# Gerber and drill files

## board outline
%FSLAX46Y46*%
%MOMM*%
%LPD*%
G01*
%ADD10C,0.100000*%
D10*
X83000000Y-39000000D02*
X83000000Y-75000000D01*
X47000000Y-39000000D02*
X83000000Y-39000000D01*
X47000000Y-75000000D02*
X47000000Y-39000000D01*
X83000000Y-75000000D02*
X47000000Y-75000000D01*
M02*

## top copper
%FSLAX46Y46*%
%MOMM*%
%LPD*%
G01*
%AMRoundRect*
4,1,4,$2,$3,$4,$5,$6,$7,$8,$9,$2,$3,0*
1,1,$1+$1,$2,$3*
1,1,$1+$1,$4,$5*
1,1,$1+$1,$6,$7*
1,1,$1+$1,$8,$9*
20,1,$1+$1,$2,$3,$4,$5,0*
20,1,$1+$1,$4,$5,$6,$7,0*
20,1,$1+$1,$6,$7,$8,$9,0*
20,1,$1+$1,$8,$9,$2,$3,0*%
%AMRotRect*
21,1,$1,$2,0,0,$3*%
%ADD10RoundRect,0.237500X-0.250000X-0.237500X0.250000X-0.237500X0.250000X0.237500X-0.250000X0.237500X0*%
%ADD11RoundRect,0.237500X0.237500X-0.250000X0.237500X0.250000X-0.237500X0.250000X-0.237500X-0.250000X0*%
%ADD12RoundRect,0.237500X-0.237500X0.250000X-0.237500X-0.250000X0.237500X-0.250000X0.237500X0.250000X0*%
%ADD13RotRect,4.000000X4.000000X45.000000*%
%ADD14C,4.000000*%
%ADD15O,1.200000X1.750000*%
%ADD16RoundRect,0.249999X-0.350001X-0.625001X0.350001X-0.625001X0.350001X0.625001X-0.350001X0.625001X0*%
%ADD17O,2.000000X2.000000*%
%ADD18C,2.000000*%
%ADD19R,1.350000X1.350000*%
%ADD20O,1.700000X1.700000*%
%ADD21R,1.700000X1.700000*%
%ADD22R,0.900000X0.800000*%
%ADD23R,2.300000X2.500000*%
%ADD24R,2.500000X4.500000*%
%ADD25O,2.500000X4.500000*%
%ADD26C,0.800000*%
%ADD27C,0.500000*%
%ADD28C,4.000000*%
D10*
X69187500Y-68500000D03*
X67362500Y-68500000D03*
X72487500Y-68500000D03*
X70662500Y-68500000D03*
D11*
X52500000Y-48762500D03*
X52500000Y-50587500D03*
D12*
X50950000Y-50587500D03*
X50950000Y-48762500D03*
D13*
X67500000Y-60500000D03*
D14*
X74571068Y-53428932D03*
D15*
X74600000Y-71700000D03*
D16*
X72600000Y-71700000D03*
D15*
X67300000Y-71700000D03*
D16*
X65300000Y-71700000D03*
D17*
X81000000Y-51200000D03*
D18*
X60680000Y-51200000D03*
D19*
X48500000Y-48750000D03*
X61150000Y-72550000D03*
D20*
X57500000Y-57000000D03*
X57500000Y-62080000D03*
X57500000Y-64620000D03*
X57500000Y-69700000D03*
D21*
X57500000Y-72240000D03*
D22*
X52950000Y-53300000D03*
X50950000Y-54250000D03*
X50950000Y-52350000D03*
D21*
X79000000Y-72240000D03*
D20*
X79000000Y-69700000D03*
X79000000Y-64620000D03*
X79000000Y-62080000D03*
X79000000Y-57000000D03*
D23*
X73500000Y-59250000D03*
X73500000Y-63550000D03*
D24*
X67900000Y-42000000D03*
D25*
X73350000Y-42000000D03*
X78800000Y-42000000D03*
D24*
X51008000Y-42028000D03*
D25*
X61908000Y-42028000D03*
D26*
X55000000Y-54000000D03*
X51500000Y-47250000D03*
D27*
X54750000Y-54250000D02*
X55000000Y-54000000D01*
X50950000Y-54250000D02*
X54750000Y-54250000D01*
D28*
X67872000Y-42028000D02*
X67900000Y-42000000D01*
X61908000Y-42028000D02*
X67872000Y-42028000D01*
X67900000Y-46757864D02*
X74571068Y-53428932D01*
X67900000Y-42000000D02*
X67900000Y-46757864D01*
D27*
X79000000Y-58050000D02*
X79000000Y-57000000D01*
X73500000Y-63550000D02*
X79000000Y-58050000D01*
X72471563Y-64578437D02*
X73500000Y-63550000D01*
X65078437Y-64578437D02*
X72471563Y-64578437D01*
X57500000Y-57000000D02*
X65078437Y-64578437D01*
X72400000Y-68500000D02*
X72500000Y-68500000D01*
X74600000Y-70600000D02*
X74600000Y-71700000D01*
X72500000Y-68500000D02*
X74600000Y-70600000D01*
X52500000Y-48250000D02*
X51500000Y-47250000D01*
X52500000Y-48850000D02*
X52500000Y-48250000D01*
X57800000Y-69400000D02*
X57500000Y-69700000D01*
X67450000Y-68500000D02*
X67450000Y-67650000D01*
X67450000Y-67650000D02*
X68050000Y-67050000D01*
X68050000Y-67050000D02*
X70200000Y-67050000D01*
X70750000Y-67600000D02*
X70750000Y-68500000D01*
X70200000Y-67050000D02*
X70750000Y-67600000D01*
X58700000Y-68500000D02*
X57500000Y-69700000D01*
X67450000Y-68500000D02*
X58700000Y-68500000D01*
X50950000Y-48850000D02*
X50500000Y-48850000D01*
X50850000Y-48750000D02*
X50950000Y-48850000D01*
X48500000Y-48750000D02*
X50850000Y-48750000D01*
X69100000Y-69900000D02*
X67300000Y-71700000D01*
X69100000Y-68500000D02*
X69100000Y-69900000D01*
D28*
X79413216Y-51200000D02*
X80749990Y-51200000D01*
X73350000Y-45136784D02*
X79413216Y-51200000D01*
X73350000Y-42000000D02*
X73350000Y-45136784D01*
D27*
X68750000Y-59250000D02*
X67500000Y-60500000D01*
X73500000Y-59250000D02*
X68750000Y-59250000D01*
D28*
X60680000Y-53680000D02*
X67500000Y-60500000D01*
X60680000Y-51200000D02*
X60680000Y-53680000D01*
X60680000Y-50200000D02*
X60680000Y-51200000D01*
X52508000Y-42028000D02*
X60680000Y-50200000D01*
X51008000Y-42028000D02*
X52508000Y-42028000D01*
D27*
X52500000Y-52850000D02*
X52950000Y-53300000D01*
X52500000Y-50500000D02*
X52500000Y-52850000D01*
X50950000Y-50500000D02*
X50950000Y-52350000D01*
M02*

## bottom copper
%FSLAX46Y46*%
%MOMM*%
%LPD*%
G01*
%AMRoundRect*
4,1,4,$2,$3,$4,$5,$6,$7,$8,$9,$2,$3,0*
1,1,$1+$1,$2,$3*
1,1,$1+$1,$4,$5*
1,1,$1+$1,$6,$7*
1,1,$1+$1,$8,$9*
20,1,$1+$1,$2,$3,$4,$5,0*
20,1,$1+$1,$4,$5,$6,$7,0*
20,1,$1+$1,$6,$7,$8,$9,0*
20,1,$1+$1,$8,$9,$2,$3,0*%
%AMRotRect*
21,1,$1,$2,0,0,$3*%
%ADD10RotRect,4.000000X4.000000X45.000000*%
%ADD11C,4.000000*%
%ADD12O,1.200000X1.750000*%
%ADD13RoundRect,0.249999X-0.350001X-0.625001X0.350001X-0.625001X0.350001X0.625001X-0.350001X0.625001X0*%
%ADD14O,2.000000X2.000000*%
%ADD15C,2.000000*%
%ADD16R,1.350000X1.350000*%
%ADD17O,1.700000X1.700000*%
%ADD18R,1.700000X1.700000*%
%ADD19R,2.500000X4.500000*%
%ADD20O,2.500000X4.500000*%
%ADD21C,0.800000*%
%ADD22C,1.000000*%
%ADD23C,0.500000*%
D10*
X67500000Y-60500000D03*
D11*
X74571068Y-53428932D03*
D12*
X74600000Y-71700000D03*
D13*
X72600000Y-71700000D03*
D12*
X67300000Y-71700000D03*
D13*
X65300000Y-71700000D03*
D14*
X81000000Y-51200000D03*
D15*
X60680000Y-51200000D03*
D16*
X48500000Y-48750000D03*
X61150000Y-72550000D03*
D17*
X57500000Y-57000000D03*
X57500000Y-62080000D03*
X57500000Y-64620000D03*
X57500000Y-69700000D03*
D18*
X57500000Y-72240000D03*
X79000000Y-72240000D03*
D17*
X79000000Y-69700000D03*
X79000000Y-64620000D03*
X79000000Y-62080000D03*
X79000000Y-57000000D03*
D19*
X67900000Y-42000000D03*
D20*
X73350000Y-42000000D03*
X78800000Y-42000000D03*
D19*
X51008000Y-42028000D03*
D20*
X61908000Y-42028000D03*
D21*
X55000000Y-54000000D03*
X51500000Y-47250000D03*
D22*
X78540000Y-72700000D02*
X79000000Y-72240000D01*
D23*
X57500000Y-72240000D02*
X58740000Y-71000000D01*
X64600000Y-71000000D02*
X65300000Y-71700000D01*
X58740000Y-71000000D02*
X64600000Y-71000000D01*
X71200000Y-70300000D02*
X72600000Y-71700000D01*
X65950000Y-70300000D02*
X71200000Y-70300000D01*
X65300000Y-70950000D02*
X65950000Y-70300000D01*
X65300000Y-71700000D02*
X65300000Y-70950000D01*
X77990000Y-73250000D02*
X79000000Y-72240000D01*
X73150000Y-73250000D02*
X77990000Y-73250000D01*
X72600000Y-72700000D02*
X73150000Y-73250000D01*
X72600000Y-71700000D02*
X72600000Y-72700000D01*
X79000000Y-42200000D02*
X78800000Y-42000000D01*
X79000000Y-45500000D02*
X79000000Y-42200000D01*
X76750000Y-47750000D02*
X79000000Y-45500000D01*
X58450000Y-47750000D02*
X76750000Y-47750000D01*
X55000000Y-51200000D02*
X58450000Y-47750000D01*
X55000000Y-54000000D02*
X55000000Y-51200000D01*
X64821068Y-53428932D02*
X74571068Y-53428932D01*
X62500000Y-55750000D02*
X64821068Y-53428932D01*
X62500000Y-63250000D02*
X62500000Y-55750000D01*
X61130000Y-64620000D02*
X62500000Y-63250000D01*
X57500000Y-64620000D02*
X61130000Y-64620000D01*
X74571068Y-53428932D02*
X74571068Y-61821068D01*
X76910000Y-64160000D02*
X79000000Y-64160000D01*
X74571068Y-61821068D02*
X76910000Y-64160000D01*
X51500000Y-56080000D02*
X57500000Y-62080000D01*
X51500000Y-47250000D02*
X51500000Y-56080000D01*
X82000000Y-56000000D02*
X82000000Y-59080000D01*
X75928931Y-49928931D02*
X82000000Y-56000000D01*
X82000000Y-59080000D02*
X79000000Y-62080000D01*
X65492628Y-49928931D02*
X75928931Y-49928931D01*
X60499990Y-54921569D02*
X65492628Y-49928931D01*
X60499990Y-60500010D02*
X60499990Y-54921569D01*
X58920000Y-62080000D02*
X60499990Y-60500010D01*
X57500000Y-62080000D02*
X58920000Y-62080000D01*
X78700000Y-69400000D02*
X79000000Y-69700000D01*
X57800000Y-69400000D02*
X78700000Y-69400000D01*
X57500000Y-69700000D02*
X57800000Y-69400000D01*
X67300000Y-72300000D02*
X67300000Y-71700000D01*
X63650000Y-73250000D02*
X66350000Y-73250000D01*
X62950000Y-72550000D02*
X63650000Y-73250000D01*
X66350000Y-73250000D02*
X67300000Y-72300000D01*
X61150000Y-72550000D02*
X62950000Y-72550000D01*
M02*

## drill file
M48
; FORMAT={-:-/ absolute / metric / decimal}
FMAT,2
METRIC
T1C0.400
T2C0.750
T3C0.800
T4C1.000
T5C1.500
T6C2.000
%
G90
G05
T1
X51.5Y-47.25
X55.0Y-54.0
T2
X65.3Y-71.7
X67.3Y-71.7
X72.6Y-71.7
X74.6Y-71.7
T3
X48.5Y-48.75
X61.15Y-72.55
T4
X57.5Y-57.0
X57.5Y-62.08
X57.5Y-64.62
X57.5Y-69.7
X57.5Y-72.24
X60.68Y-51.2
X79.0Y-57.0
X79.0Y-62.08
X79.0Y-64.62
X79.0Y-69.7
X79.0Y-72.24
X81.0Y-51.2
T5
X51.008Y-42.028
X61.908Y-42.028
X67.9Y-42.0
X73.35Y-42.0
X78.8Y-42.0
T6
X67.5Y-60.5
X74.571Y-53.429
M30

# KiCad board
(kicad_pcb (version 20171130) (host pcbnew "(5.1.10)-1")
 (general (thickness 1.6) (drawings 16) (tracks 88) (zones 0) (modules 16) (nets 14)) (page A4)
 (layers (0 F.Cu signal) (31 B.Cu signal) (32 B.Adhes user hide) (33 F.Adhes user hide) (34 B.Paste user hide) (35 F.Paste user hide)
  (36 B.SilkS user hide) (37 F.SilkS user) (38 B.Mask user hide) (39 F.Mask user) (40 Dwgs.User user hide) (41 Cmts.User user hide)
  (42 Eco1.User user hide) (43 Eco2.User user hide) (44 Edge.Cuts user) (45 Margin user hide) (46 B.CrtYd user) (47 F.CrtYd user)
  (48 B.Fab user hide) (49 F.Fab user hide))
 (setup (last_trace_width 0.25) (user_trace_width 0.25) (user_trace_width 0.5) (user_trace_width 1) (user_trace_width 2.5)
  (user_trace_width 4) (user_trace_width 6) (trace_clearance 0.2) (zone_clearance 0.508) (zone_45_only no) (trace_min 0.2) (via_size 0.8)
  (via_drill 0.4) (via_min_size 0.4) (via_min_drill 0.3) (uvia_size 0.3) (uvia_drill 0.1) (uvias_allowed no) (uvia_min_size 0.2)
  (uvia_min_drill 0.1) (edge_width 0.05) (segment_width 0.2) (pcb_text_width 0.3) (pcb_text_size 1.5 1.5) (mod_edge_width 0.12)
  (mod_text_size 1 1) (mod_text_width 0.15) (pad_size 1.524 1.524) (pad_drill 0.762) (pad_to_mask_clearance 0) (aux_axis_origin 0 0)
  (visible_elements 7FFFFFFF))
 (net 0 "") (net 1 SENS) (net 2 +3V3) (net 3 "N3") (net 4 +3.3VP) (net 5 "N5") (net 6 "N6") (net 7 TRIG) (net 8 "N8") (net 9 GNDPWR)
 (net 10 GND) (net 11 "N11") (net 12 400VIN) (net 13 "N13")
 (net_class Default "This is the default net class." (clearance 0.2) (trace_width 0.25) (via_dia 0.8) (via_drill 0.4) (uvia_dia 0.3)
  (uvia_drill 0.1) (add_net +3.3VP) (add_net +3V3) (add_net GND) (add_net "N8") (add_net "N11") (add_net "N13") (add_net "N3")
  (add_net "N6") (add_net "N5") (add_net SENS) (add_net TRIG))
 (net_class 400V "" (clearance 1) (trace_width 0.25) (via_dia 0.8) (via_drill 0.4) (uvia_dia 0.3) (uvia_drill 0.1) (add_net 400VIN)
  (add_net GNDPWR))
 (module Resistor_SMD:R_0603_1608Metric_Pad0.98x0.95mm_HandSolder (layer F.Cu) (at 68.275 68.5)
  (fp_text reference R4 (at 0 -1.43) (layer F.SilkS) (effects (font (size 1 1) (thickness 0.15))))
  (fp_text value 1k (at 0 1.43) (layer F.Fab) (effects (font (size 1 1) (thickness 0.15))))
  (pad 2 smd roundrect (at 0.9125 0) (size 0.975 0.95) (layers F.Cu F.Paste F.Mask) (roundrect_rratio 0.25) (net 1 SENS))
  (pad 1 smd roundrect (at -0.9125 0) (size 0.975 0.95) (layers F.Cu F.Paste F.Mask) (roundrect_rratio 0.25) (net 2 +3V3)))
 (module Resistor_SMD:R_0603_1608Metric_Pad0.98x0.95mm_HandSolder (layer F.Cu) (at 71.575 68.5)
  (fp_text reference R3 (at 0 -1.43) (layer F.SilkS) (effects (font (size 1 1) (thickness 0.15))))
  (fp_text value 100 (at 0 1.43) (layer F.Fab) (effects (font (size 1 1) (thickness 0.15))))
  (pad 2 smd roundrect (at 0.9125 0) (size 0.975 0.95) (layers F.Cu F.Paste F.Mask) (roundrect_rratio 0.25) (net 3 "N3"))
  (pad 1 smd roundrect (at -0.9125 0) (size 0.975 0.95) (layers F.Cu F.Paste F.Mask) (roundrect_rratio 0.25) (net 2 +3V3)))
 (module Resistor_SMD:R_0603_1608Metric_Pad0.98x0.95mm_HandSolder (layer F.Cu) (at 52.5 49.675 90)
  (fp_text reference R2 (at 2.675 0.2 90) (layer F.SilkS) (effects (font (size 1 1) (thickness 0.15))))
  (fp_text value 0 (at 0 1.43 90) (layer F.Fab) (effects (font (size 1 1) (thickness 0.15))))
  (pad 2 smd roundrect (at 0.9125 0 90) (size 0.975 0.95) (layers F.Cu F.Paste F.Mask) (roundrect_rratio 0.25) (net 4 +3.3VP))
  (pad 1 smd roundrect (at -0.9125 0 90) (size 0.975 0.95) (layers F.Cu F.Paste F.Mask) (roundrect_rratio 0.25) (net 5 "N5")))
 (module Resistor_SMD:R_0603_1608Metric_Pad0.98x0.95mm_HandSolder (layer F.Cu) (at 50.95 49.675 270)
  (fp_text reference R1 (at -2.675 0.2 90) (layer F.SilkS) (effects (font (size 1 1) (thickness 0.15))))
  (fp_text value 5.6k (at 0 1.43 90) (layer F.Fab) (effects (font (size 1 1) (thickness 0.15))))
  (pad 2 smd roundrect (at 0.9125 0 270) (size 0.975 0.95) (layers F.Cu F.Paste F.Mask) (roundrect_rratio 0.25) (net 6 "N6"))
  (pad 1 smd roundrect (at -0.9125 0 270) (size 0.975 0.95) (layers F.Cu F.Paste F.Mask) (roundrect_rratio 0.25) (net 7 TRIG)))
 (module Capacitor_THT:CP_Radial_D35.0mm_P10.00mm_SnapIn (layer B.Cu) (at 67.5 60.5 45)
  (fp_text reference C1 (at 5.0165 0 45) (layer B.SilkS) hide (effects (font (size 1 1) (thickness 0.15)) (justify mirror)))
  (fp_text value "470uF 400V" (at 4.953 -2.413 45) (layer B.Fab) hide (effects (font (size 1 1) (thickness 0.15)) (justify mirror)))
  (pad 1 thru_hole rect (at 0 0 45) (size 4 4) (drill 2) (layers *.Cu *.Mask) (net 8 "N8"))
  (pad 2 thru_hole circle (at 10 0 45) (size 4 4) (drill 2) (layers *.Cu *.Mask) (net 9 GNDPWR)))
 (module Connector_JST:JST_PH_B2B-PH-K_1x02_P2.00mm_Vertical (layer F.Cu) (at 72.6 71.7)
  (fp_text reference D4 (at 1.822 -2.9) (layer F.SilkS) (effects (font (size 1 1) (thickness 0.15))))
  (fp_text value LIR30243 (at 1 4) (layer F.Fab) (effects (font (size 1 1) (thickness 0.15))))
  (pad 2 thru_hole oval (at 2 0) (size 1.2 1.75) (drill 0.75) (layers *.Cu *.Mask) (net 3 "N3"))
  (pad 1 thru_hole roundrect (at 0 0) (size 1.2 1.75) (drill 0.75) (layers *.Cu *.Mask) (roundrect_rratio 0.2083325) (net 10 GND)))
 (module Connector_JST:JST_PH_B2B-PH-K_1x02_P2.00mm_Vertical (layer F.Cu) (at 65.3 71.7)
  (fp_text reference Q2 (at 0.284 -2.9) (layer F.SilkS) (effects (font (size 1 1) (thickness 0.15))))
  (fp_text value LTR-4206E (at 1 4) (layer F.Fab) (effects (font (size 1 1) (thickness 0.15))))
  (pad 2 thru_hole oval (at 2 0) (size 1.2 1.75) (drill 0.75) (layers *.Cu *.Mask) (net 1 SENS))
  (pad 1 thru_hole roundrect (at 0 0) (size 1.2 1.75) (drill 0.75) (layers *.Cu *.Mask) (roundrect_rratio 0.2083325) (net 10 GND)))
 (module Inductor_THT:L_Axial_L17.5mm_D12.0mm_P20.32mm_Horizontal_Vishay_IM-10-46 (layer F.Cu) (at 60.68 51.2)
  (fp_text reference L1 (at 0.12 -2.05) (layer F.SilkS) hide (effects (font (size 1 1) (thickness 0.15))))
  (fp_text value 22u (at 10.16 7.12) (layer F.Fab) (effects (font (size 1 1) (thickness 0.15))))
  (pad 2 thru_hole oval (at 20.32 0) (size 2 2) (drill 1) (layers *.Cu *.Mask) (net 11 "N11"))
  (pad 1 thru_hole circle (at 0 0) (size 2 2) (drill 1) (layers *.Cu *.Mask) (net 8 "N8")))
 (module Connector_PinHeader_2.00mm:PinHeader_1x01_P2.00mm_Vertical (layer F.Cu) (at 48.5 48.75 180)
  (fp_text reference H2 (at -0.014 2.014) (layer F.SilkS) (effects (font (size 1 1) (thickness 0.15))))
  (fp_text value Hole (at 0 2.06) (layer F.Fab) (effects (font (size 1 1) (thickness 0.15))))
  (pad 1 thru_hole rect (at 0 0 180) (size 1.35 1.35) (drill 0.8) (layers *.Cu *.Mask) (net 7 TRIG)))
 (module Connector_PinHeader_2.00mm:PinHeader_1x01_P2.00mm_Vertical (layer F.Cu) (at 61.15 72.55 180)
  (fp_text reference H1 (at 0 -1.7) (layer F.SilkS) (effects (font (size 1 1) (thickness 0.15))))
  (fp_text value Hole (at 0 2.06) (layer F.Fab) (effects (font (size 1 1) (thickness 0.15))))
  (pad 1 thru_hole rect (at 0 0 180) (size 1.35 1.35) (drill 0.8) (layers *.Cu *.Mask) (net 1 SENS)))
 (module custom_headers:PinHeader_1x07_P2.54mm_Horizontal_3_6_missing (layer F.Cu) (at 57.5 72.24 180)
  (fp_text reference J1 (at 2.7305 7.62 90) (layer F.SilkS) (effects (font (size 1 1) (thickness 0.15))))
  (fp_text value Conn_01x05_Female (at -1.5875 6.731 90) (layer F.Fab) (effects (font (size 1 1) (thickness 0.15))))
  (pad 5 thru_hole oval (at 0 15.24 180) (size 1.7 1.7) (drill 1) (layers *.Cu *.Mask) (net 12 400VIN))
  (pad 4 thru_hole oval (at 0 10.16 180) (size 1.7 1.7) (drill 1) (layers *.Cu *.Mask) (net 4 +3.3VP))
  (pad 3 thru_hole oval (at 0 7.62 180) (size 1.7 1.7) (drill 1) (layers *.Cu *.Mask) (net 9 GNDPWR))
  (pad 2 thru_hole oval (at 0 2.54 180) (size 1.7 1.7) (drill 1) (layers *.Cu *.Mask) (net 2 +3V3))
  (pad 1 thru_hole rect (at 0 0 180) (size 1.7 1.7) (drill 1) (layers *.Cu *.Mask) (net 10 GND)))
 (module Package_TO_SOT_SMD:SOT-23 (layer F.Cu) (at 51.95 53.3)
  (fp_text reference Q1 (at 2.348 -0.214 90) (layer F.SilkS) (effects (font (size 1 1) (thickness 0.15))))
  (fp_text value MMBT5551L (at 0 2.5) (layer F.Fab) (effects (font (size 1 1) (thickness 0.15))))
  (pad 3 smd rect (at 1 0) (size 0.9 0.8) (layers F.Cu F.Paste F.Mask) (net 5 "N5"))
  (pad 2 smd rect (at -1 0.95) (size 0.9 0.8) (layers F.Cu F.Paste F.Mask) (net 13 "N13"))
  (pad 1 smd rect (at -1 -0.95) (size 0.9 0.8) (layers F.Cu F.Paste F.Mask) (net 6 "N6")))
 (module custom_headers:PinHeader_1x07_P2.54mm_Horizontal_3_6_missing (layer B.Cu) (at 79 72.24)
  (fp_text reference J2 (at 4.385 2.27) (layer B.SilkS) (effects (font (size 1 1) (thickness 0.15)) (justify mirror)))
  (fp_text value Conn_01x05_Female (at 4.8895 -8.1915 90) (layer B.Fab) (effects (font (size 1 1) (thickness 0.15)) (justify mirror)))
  (pad 1 thru_hole rect (at 0 0) (size 1.7 1.7) (drill 1) (layers *.Cu *.Mask) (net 10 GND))
  (pad 2 thru_hole oval (at 0 -2.54) (size 1.7 1.7) (drill 1) (layers *.Cu *.Mask) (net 2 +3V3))
  (pad 3 thru_hole oval (at 0 -7.62) (size 1.7 1.7) (drill 1) (layers *.Cu *.Mask) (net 9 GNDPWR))
  (pad 4 thru_hole oval (at 0 -10.16) (size 1.7 1.7) (drill 1) (layers *.Cu *.Mask) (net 4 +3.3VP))
  (pad 5 thru_hole oval (at 0 -15.24) (size 1.7 1.7) (drill 1) (layers *.Cu *.Mask) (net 12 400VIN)))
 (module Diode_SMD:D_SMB (layer F.Cu) (at 73.5 61.4 270)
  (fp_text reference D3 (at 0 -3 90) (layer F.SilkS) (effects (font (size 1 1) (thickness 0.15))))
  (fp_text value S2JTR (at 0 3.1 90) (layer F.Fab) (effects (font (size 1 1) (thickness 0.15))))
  (pad 1 smd rect (at -2.15 0 270) (size 2.5 2.3) (layers F.Cu F.Paste F.Mask) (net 8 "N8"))
  (pad 2 smd rect (at 2.15 0 270) (size 2.5 2.3) (layers F.Cu F.Paste F.Mask) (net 12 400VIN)))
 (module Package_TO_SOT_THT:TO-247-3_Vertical (layer F.Cu) (at 67.9 42)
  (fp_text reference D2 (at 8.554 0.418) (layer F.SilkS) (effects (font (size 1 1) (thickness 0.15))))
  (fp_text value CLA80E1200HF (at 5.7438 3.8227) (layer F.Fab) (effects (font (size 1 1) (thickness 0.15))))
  (pad 1 thru_hole rect (at 0 0) (size 2.5 4.5) (drill 1.5) (layers *.Cu *.Mask) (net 9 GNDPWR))
  (pad 2 thru_hole oval (at 5.45 0) (size 2.5 4.5) (drill 1.5) (layers *.Cu *.Mask) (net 11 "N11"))
  (pad 3 thru_hole oval (at 10.9 0) (size 2.5 4.5) (drill 1.5) (layers *.Cu *.Mask) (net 13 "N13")))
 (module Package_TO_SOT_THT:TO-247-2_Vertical (layer F.Cu) (at 51.008 42.028)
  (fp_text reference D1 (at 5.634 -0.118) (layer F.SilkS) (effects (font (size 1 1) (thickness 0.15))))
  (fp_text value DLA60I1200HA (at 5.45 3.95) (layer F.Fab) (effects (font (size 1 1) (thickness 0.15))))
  (pad 1 thru_hole rect (at 0 0) (size 2.5 4.5) (drill 1.5) (layers *.Cu *.Mask) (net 8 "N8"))
  (pad 2 thru_hole oval (at 10.9 0) (size 2.5 4.5) (drill 1.5) (layers *.Cu *.Mask) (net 9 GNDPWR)))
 (gr_line (start 83 39) (end 83 75) (layer Edge.Cuts) (width 0.1))
 (gr_line (start 47 39) (end 83 39) (layer Edge.Cuts) (width 0.1))
 (gr_line (start 47 75) (end 47 39) (layer Edge.Cuts) (width 0.1))
 (gr_line (start 83 75) (end 47 75) (layer Edge.Cuts) (width 0.1))
 (segment (start 78.54 72.7) (end 79 72.24) (width 1) (layer B.Cu) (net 10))
 (segment (start 57.5 72.24) (end 58.74 71) (width 0.5) (layer B.Cu) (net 10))
 (segment (start 64.6 71) (end 65.3 71.7) (width 0.5) (layer B.Cu) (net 10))
 (segment (start 58.74 71) (end 64.6 71) (width 0.5) (layer B.Cu) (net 10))
 (segment (start 71.2 70.3) (end 72.6 71.7) (width 0.5) (layer B.Cu) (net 10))
 (segment (start 65.95 70.3) (end 71.2 70.3) (width 0.5) (layer B.Cu) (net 10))
 (segment (start 65.3 70.95) (end 65.95 70.3) (width 0.5) (layer B.Cu) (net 10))
 (segment (start 65.3 71.7) (end 65.3 70.95) (width 0.5) (layer B.Cu) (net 10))
 (segment (start 77.99 73.25) (end 79 72.24) (width 0.5) (layer B.Cu) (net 10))
 (segment (start 73.15 73.25) (end 77.99 73.25) (width 0.5) (layer B.Cu) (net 10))
 (segment (start 72.6 72.7) (end 73.15 73.25) (width 0.5) (layer B.Cu) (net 10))
 (segment (start 72.6 71.7) (end 72.6 72.7) (width 0.5) (layer B.Cu) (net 10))
 (via (at 55 54) (size 0.8) (drill 0.4) (layers F.Cu B.Cu) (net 13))
 (segment (start 79 42.2) (end 78.8 42) (width 0.5) (layer B.Cu) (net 13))
 (segment (start 79 45.5) (end 79 42.2) (width 0.5) (layer B.Cu) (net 13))
 (segment (start 76.75 47.75) (end 79 45.5) (width 0.5) (layer B.Cu) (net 13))
 (segment (start 58.45 47.75) (end 76.75 47.75) (width 0.5) (layer B.Cu) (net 13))
 (segment (start 55 51.2) (end 58.45 47.75) (width 0.5) (layer B.Cu) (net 13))
 (segment (start 55 54) (end 55 51.2) (width 0.5) (layer B.Cu) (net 13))
 (segment (start 54.75 54.25) (end 55 54) (width 0.5) (layer F.Cu) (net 13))
 (segment (start 50.95 54.25) (end 54.75 54.25) (width 0.5) (layer F.Cu) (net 13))
 (segment (start 64.821068 53.428932) (end 74.571068 53.428932) (width 0.5) (layer B.Cu) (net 9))
 (segment (start 62.5 55.75) (end 64.821068 53.428932) (width 0.5) (layer B.Cu) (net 9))
 (segment (start 62.5 63.25) (end 62.5 55.75) (width 0.5) (layer B.Cu) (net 9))
 (segment (start 61.13 64.62) (end 62.5 63.25) (width 0.5) (layer B.Cu) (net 9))
 (segment (start 57.5 64.62) (end 61.13 64.62) (width 0.5) (layer B.Cu) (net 9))
 (segment (start 74.571068 53.428932) (end 74.571068 61.821068) (width 0.5) (layer B.Cu) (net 9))
 (segment (start 76.91 64.16) (end 79 64.16) (width 0.5) (layer B.Cu) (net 9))
 (segment (start 74.571068 61.821068) (end 76.91 64.16) (width 0.5) (layer B.Cu) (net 9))
 (segment (start 67.872 42.028) (end 67.9 42) (width 4) (layer F.Cu) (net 9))
 (segment (start 61.908 42.028) (end 67.872 42.028) (width 4) (layer F.Cu) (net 9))
 (segment (start 67.9 46.757864) (end 74.571068 53.428932) (width 4) (layer F.Cu) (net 9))
 (segment (start 67.9 42) (end 67.9 46.757864) (width 4) (layer F.Cu) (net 9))
 (segment (start 79 58.05) (end 79 57) (width 0.5) (layer F.Cu) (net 12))
 (segment (start 73.5 63.55) (end 79 58.05) (width 0.5) (layer F.Cu) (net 12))
 (segment (start 72.471563 64.578437) (end 73.5 63.55) (width 0.5) (layer F.Cu) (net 12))
 (segment (start 65.078437 64.578437) (end 72.471563 64.578437) (width 0.5) (layer F.Cu) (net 12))
 (segment (start 57.5 57) (end 65.078437 64.578437) (width 0.5) (layer F.Cu) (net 12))
 (segment (start 72.4 68.5) (end 72.5 68.5) (width 0.5) (layer F.Cu) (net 3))
 (segment (start 74.6 70.6) (end 74.6 71.7) (width 0.5) (layer F.Cu) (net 3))
 (segment (start 72.5 68.5) (end 74.6 70.6) (width 0.5) (layer F.Cu) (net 3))
 (via (at 51.5 47.25) (size 0.8) (drill 0.4) (layers F.Cu B.Cu) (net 4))
 (segment (start 51.5 56.08) (end 57.5 62.08) (width 0.5) (layer B.Cu) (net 4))
 (segment (start 51.5 47.25) (end 51.5 56.08) (width 0.5) (layer B.Cu) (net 4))
 (segment (start 82 56) (end 82 59.08) (width 0.5) (layer B.Cu) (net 4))
 (segment (start 75.928931 49.928931) (end 82 56) (width 0.5) (layer B.Cu) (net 4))
 (segment (start 82 59.08) (end 79 62.08) (width 0.5) (layer B.Cu) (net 4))
 (segment (start 65.492628 49.928931) (end 75.928931 49.928931) (width 0.5) (layer B.Cu) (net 4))
 (segment (start 60.49999 54.921569) (end 65.492628 49.928931) (width 0.5) (layer B.Cu) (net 4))
 (segment (start 60.49999 60.50001) (end 60.49999 54.921569) (width 0.5) (layer B.Cu) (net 4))
 (segment (start 58.92 62.08) (end 60.49999 60.50001) (width 0.5) (layer B.Cu) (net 4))
 (segment (start 57.5 62.08) (end 58.92 62.08) (width 0.5) (layer B.Cu) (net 4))
 (segment (start 52.5 48.25) (end 51.5 47.25) (width 0.5) (layer F.Cu) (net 4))
 (segment (start 52.5 48.85) (end 52.5 48.25) (width 0.5) (layer F.Cu) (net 4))
 (segment (start 57.8 69.4) (end 57.5 69.7) (width 0.5) (layer F.Cu) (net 2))
 (segment (start 67.45 68.5) (end 67.45 67.65) (width 0.5) (layer F.Cu) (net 2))
 (segment (start 67.45 67.65) (end 68.05 67.05) (width 0.5) (layer F.Cu) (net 2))
 (segment (start 68.05 67.05) (end 70.2 67.05) (width 0.5) (layer F.Cu) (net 2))
 (segment (start 70.75 67.6) (end 70.75 68.5) (width 0.5) (layer F.Cu) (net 2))
 (segment (start 70.2 67.05) (end 70.75 67.6) (width 0.5) (layer F.Cu) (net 2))
 (segment (start 58.7 68.5) (end 57.5 69.7) (width 0.5) (layer F.Cu) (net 2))
 (segment (start 67.45 68.5) (end 58.7 68.5) (width 0.5) (layer F.Cu) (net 2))
 (segment (start 78.7 69.4) (end 79 69.7) (width 0.5) (layer B.Cu) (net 2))
 (segment (start 57.8 69.4) (end 78.7 69.4) (width 0.5) (layer B.Cu) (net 2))
 (segment (start 57.5 69.7) (end 57.8 69.4) (width 0.5) (layer B.Cu) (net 2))
 (segment (start 50.95 48.85) (end 50.5 48.85) (width 0.5) (layer F.Cu) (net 7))
 (segment (start 50.85 48.75) (end 50.95 48.85) (width 0.5) (layer F.Cu) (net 7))
 (segment (start 48.5 48.75) (end 50.85 48.75) (width 0.5) (layer F.Cu) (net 7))
 (segment (start 69.1 69.9) (end 67.3 71.7) (width 0.5) (layer F.Cu) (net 1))
 (segment (start 69.1 68.5) (end 69.1 69.9) (width 0.5) (layer F.Cu) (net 1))
 (segment (start 67.3 72.3) (end 67.3 71.7) (width 0.5) (layer B.Cu) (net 1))
 (segment (start 63.65 73.25) (end 66.35 73.25) (width 0.5) (layer B.Cu) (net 1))
 (segment (start 62.95 72.55) (end 63.65 73.25) (width 0.5) (layer B.Cu) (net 1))
 (segment (start 66.35 73.25) (end 67.3 72.3) (width 0.5) (layer B.Cu) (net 1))
 (segment (start 61.15 72.55) (end 62.95 72.55) (width 0.5) (layer B.Cu) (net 1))
 (segment (start 79.413216 51.2) (end 80.74999 51.2) (width 4) (layer F.Cu) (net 11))
 (segment (start 73.35 45.136784) (end 79.413216 51.2) (width 4) (layer F.Cu) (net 11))
 (segment (start 73.35 42) (end 73.35 45.136784) (width 4) (layer F.Cu) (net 11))
 (segment (start 68.75 59.25) (end 67.5 60.5) (width 0.5) (layer F.Cu) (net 8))
 (segment (start 73.5 59.25) (end 68.75 59.25) (width 0.5) (layer F.Cu) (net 8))
 (segment (start 60.68 53.68) (end 67.5 60.5) (width 4) (layer F.Cu) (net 8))
 (segment (start 60.68 51.2) (end 60.68 53.68) (width 4) (layer F.Cu) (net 8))
 (segment (start 60.68 50.2) (end 60.68 51.2) (width 4) (layer F.Cu) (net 8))
 (segment (start 52.508 42.028) (end 60.68 50.2) (width 4) (layer F.Cu) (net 8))
 (segment (start 51.008 42.028) (end 52.508 42.028) (width 4) (layer F.Cu) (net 8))
 (segment (start 52.5 52.85) (end 52.95 53.3) (width 0.5) (layer F.Cu) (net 5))
 (segment (start 52.5 50.5) (end 52.5 52.85) (width 0.5) (layer F.Cu) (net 5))
 (segment (start 50.95 50.5) (end 50.95 52.35) (width 0.5) (layer F.Cu) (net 6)))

